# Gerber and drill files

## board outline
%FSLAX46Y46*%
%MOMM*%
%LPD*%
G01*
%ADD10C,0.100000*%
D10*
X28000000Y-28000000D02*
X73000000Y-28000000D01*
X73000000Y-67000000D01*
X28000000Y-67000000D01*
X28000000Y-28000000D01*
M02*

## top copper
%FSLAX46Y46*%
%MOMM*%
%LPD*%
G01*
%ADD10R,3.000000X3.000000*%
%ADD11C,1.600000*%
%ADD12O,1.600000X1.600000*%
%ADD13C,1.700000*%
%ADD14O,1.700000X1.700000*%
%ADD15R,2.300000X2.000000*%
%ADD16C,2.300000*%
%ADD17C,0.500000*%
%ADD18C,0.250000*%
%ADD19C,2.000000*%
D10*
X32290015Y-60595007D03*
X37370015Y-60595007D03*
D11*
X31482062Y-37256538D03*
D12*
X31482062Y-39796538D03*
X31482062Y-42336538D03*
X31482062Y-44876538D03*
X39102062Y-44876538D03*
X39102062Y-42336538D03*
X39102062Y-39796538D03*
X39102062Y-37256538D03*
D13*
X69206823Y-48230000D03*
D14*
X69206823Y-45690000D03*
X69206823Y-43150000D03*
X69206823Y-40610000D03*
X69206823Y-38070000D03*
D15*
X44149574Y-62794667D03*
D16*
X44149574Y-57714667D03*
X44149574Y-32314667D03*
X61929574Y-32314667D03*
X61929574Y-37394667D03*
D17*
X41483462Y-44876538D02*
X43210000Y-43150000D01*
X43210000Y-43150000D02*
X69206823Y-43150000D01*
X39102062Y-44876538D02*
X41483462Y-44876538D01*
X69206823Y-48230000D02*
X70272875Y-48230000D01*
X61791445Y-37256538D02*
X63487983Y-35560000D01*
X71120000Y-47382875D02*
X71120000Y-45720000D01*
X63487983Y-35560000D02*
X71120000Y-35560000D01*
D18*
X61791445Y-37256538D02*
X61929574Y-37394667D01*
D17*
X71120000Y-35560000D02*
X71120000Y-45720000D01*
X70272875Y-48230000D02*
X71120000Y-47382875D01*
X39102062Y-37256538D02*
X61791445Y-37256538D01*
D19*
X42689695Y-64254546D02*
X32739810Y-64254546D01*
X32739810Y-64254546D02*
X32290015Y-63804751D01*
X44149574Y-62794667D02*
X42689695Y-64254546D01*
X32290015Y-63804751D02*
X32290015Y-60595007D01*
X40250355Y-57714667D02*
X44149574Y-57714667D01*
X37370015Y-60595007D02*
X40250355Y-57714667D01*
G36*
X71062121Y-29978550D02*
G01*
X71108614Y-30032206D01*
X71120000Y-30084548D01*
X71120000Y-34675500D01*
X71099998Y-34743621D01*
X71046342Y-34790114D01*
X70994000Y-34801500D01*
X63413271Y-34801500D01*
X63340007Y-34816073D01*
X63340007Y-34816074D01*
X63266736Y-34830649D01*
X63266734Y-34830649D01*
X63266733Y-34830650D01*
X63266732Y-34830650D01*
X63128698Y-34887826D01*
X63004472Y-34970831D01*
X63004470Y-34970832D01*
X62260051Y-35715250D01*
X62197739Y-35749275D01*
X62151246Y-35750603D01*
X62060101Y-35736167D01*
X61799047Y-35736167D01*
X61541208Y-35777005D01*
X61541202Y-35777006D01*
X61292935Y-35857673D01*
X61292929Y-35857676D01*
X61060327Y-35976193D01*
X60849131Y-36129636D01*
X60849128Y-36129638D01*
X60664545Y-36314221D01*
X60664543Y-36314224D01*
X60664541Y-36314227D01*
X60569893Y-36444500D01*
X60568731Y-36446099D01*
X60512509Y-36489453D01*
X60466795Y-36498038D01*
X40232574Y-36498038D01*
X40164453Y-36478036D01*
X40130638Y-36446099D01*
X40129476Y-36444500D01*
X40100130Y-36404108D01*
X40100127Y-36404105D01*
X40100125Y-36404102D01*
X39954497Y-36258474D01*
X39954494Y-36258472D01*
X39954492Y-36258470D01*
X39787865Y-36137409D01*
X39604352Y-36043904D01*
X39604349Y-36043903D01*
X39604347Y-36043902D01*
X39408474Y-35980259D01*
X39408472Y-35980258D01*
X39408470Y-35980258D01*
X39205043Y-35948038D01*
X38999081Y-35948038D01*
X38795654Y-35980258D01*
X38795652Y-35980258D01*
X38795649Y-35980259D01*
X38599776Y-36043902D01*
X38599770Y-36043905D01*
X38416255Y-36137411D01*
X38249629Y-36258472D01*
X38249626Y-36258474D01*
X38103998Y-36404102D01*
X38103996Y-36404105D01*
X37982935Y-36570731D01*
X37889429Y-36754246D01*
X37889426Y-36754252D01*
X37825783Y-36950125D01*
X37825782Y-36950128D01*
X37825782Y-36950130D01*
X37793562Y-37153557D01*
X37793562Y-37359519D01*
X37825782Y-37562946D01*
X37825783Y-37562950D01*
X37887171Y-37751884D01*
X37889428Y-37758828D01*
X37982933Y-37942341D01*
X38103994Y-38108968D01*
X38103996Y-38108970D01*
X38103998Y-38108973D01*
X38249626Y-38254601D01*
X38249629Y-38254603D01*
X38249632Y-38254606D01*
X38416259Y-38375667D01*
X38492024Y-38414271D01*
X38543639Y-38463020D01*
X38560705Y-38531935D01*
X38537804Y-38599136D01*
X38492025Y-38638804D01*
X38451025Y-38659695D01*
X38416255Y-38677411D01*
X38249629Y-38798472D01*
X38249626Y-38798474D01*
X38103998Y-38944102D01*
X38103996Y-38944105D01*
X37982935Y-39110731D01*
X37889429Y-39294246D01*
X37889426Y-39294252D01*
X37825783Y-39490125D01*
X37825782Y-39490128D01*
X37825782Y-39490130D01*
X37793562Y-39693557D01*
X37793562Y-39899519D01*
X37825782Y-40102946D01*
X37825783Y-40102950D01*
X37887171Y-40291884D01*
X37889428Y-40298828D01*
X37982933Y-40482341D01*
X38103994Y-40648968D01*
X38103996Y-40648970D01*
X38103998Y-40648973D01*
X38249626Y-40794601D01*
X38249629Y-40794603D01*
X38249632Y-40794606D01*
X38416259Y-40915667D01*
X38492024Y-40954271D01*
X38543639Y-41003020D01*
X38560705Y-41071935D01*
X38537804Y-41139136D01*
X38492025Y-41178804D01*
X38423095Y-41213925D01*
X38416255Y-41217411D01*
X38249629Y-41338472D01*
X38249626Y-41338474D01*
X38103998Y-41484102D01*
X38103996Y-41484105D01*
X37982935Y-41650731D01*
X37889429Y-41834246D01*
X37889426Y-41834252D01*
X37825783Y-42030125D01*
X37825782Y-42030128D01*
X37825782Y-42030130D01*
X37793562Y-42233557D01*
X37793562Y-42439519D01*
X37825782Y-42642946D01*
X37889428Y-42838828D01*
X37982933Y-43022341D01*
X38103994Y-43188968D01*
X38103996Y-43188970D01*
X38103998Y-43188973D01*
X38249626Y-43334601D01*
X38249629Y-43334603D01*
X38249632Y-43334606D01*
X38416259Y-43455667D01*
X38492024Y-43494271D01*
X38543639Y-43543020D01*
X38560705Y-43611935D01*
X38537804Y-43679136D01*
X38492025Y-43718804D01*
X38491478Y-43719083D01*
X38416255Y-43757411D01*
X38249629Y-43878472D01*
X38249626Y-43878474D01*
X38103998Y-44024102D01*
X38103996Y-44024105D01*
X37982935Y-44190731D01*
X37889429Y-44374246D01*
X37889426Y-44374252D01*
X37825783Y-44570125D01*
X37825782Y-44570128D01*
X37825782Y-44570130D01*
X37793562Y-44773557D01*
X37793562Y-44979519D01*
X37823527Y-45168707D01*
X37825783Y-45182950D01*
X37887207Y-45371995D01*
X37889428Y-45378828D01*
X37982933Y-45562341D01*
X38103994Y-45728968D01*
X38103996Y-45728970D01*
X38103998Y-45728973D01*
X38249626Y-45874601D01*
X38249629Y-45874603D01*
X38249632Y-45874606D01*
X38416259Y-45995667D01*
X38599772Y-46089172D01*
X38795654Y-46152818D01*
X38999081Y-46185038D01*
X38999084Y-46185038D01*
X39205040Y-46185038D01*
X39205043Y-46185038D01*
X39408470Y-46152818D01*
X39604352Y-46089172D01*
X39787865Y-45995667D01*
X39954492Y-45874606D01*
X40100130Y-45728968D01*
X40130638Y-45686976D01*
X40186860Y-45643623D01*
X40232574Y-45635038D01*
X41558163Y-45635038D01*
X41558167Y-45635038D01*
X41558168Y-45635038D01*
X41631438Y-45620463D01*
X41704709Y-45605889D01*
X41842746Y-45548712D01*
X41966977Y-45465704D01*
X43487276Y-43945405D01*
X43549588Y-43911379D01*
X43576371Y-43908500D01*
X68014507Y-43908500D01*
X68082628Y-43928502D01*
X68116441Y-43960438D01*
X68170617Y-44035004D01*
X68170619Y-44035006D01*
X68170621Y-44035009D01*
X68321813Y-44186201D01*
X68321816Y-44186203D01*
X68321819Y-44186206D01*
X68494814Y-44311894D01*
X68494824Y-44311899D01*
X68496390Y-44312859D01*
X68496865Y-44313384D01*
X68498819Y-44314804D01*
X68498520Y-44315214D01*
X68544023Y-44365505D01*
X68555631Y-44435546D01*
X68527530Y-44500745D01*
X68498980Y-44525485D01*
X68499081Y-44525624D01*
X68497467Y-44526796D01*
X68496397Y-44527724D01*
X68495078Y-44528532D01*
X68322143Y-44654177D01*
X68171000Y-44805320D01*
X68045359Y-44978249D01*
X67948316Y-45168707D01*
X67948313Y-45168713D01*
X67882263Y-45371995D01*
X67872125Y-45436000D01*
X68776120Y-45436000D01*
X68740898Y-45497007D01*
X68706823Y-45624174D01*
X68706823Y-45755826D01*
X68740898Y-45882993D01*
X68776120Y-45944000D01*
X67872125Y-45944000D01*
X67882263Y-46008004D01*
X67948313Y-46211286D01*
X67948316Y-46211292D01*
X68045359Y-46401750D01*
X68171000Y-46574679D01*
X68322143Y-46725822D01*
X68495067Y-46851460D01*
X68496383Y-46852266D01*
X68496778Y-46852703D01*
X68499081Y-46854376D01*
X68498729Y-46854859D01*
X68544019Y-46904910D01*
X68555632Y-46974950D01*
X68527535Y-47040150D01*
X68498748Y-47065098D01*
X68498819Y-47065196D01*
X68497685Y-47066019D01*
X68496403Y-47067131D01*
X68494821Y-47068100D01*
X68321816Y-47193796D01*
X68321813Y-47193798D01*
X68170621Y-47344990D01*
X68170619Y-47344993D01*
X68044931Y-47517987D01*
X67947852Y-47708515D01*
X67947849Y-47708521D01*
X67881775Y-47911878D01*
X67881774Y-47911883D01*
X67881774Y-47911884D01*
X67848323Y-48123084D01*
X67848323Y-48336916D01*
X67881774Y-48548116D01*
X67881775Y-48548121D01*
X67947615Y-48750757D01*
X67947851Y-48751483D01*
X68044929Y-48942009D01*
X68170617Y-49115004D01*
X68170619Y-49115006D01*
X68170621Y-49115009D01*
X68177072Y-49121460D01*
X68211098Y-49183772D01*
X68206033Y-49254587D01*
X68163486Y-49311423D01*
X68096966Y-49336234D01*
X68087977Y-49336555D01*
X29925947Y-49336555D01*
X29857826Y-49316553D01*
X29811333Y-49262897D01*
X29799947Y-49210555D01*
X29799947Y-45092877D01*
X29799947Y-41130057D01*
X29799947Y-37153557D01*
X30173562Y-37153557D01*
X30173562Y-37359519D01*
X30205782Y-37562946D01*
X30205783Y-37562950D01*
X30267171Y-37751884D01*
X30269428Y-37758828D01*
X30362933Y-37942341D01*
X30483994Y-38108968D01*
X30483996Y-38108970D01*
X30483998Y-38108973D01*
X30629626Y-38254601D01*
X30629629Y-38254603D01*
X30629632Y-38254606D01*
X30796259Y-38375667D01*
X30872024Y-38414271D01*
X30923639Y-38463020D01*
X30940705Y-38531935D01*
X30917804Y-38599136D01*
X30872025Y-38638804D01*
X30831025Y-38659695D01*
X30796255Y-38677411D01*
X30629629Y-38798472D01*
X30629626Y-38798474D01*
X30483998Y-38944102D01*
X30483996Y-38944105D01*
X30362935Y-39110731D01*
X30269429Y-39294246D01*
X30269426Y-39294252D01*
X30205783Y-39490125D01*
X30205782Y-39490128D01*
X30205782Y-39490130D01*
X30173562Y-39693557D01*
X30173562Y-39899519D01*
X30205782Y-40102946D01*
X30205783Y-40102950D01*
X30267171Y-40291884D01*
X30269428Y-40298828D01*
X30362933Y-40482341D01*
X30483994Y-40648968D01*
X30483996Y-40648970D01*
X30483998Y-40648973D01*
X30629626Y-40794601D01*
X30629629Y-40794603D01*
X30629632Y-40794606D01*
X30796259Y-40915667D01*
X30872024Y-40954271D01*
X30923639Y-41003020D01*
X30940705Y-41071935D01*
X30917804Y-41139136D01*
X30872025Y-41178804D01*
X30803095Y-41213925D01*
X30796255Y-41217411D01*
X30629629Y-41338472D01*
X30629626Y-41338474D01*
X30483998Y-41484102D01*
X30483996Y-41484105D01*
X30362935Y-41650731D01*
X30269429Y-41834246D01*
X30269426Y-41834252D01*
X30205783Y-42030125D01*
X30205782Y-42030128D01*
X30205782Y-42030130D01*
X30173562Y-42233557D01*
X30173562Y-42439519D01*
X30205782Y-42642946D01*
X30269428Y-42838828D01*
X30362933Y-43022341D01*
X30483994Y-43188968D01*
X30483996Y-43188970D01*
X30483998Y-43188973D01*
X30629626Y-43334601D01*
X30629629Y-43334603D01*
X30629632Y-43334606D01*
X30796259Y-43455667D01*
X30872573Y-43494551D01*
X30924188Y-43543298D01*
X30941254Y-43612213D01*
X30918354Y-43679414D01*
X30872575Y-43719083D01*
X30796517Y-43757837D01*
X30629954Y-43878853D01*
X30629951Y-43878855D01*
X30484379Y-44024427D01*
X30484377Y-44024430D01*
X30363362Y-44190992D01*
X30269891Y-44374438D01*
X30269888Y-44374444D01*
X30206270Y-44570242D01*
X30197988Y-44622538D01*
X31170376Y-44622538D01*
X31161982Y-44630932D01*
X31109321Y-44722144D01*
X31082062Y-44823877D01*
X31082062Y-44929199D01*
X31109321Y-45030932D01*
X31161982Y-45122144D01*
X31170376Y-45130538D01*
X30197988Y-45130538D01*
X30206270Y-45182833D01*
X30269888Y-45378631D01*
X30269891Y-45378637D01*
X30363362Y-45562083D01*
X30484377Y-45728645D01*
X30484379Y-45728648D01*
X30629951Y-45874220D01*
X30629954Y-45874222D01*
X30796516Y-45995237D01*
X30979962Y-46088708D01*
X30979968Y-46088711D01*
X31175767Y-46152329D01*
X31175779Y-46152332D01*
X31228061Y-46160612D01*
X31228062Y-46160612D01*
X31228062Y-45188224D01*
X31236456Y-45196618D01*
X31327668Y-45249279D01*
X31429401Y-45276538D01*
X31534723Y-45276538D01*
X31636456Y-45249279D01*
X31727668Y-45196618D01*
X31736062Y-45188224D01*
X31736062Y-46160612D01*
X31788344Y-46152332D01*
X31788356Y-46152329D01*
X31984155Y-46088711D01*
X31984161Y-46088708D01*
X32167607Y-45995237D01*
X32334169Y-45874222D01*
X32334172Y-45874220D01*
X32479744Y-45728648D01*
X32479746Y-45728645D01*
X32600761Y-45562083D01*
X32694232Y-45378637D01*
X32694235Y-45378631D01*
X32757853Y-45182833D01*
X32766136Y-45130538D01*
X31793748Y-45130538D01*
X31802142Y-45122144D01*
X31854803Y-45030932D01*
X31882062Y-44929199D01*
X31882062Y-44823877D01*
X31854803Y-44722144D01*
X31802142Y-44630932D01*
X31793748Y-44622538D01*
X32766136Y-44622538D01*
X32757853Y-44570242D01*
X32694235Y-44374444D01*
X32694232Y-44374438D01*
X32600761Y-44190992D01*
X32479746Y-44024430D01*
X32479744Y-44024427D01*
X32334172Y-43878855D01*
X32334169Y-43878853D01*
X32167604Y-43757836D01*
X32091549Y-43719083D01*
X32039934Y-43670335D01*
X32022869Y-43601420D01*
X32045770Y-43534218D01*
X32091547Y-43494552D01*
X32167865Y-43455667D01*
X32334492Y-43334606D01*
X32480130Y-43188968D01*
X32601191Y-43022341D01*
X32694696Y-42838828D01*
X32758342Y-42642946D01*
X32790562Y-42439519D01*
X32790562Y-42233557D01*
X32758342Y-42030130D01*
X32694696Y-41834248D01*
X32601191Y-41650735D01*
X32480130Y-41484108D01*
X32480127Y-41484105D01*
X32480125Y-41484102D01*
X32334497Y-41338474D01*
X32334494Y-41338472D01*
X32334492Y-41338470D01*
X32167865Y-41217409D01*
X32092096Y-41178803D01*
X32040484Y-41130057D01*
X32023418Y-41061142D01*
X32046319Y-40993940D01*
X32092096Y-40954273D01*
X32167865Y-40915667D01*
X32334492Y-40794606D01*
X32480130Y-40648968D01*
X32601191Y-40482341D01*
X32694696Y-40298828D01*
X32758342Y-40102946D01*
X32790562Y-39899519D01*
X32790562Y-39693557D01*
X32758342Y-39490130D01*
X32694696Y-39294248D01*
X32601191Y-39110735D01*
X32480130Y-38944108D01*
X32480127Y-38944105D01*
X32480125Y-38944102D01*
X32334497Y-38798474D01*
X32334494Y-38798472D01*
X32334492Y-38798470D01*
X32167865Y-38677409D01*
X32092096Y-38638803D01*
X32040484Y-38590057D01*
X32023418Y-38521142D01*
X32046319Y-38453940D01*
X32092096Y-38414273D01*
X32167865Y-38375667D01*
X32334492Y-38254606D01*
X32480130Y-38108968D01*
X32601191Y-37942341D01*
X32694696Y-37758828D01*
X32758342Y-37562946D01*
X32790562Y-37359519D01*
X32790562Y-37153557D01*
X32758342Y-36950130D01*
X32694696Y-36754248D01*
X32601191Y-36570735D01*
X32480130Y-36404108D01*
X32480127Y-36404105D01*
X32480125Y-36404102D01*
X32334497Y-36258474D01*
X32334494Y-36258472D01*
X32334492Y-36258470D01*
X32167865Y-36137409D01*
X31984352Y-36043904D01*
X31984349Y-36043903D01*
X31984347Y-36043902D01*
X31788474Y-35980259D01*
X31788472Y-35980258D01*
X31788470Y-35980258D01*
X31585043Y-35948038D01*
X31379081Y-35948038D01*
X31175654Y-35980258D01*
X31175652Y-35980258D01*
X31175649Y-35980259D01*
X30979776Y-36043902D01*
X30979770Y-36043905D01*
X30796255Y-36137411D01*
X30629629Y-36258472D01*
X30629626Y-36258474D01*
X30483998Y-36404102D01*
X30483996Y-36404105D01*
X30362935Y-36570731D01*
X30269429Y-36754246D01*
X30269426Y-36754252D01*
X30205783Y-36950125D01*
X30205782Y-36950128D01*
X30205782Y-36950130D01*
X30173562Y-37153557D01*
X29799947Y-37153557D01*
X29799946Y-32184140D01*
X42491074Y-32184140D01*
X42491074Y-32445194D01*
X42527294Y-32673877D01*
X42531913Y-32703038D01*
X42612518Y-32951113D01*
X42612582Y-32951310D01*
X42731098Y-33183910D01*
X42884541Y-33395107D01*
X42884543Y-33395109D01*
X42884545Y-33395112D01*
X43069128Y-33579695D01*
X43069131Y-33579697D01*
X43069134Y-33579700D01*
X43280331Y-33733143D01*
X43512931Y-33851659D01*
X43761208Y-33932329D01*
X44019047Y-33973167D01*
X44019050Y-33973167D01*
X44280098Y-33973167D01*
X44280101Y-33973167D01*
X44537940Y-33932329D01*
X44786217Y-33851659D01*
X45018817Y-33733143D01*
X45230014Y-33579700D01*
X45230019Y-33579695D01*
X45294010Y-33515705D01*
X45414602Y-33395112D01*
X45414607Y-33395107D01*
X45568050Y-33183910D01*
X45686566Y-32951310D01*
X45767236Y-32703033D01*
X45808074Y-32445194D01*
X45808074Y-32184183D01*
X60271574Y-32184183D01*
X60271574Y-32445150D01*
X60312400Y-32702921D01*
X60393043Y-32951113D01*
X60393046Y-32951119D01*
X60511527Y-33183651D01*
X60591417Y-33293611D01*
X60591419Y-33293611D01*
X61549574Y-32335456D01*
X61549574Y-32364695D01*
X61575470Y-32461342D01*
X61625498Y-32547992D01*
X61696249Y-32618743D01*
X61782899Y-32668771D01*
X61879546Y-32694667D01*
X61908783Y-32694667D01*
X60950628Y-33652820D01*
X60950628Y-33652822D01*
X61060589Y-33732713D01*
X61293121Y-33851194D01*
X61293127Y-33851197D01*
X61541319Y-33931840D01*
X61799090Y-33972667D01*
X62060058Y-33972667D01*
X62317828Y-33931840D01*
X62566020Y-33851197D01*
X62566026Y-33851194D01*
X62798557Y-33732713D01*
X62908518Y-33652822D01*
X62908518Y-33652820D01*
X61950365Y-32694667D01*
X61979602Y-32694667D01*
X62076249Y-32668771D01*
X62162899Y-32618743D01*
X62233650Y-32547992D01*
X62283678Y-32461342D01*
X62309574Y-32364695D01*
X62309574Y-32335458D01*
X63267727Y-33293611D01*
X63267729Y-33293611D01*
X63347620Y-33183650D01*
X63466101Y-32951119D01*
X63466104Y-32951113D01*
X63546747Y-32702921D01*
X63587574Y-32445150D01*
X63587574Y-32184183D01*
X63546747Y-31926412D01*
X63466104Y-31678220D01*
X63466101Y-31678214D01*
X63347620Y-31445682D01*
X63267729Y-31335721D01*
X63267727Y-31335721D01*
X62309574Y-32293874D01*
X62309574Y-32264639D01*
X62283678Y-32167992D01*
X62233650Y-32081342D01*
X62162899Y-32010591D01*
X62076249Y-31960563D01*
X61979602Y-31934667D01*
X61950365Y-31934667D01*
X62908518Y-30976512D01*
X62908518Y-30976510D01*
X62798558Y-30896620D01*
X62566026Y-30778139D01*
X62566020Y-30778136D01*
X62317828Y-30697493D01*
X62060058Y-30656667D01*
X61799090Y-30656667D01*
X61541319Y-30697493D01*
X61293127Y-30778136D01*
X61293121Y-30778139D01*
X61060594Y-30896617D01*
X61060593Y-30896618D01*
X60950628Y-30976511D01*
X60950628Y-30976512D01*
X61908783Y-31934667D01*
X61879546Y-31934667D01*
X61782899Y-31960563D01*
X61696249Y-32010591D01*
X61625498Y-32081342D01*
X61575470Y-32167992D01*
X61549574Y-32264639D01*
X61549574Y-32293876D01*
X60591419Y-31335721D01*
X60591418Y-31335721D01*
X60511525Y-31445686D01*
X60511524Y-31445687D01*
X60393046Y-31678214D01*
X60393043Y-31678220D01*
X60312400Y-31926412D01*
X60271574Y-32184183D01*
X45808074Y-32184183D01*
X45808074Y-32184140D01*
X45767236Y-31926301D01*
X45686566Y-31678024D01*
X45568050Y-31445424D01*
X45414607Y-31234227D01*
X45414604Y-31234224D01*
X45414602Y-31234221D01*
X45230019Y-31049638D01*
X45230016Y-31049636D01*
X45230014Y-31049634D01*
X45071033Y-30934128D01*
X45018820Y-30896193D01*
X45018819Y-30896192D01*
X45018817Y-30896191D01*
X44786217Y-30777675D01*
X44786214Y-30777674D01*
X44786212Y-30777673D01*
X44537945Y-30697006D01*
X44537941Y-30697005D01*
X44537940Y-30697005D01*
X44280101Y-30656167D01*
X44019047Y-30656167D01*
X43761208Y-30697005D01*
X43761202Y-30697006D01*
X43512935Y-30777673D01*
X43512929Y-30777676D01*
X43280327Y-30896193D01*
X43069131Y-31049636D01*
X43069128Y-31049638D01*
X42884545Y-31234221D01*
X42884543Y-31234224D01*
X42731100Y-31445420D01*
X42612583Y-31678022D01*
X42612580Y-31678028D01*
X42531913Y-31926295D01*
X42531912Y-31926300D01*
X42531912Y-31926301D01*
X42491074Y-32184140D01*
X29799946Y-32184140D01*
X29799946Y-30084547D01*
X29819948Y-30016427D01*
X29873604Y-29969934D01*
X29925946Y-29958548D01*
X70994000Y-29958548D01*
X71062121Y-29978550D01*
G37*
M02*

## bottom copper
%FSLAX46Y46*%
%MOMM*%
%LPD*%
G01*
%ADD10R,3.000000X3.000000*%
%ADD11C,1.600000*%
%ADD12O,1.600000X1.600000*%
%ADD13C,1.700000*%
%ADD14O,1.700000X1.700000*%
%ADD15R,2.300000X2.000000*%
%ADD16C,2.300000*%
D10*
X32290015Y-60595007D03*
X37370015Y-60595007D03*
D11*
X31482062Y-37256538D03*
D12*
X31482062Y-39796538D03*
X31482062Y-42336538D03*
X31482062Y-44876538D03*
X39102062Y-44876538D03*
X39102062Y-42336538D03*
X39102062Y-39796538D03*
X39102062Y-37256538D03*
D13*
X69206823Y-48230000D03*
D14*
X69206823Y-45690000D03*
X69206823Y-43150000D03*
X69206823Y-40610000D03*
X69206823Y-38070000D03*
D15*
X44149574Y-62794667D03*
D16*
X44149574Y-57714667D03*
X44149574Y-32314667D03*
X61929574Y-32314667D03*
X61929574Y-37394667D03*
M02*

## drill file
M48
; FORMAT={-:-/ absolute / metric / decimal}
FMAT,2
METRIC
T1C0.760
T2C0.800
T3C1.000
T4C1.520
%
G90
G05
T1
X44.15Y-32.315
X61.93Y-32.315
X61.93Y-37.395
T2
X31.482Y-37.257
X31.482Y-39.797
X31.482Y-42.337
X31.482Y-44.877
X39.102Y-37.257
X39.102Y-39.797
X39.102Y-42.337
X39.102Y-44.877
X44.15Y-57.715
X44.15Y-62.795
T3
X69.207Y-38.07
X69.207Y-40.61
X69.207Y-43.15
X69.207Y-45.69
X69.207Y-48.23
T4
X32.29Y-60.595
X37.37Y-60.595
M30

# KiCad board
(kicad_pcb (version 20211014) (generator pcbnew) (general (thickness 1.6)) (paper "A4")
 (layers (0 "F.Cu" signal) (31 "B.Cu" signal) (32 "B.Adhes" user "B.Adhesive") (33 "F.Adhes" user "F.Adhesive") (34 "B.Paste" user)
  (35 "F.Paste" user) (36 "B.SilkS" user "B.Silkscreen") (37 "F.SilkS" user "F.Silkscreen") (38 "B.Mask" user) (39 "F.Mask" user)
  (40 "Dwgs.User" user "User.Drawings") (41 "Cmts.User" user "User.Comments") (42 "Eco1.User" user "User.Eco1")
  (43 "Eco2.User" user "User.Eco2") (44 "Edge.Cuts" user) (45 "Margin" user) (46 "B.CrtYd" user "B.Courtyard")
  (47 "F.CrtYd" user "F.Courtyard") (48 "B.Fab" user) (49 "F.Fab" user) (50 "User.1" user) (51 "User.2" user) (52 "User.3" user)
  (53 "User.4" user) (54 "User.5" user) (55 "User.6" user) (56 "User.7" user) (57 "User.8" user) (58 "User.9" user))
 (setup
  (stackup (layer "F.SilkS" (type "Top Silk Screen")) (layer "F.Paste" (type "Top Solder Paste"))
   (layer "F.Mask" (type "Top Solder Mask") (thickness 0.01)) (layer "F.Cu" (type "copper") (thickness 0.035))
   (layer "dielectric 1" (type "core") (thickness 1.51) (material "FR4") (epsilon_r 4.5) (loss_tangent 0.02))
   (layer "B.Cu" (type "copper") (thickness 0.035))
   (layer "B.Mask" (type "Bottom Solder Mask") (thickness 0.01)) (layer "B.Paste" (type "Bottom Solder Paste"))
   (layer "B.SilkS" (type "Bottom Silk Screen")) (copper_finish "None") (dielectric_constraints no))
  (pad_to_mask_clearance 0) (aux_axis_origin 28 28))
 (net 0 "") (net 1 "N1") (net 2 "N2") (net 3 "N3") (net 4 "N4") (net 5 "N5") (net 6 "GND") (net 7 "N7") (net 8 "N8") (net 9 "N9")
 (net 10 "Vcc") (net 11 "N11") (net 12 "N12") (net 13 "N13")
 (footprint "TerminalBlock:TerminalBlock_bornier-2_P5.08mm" (layer "F.Cu") (at 32.290015 60.595007)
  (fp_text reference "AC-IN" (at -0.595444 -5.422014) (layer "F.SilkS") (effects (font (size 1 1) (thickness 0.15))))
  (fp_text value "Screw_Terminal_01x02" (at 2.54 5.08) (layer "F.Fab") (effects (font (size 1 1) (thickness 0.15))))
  (pad "1" thru_hole rect (at 0 0) (size 3 3) (drill 1.52) (layers *.Cu *.Mask) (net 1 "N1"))
  (pad "2" thru_hole rect (at 5.08 0) (size 3 3) (drill 1.52) (layers *.Cu *.Mask) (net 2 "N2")))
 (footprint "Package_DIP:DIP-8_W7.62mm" (layer "F.Cu") (at 31.482062 37.256538)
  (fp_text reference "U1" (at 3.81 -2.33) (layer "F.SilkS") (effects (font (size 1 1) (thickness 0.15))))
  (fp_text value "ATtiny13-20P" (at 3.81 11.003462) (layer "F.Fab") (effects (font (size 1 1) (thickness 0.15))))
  (pad "1" thru_hole circle (at 0 0) (size 1.6 1.6) (drill 0.8) (layers *.Cu *.Mask) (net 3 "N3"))
  (pad "2" thru_hole oval (at 0 2.54) (size 1.6 1.6) (drill 0.8) (layers *.Cu *.Mask) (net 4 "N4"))
  (pad "3" thru_hole oval (at 0 5.08) (size 1.6 1.6) (drill 0.8) (layers *.Cu *.Mask) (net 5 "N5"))
  (pad "4" thru_hole oval (at 0 7.62) (size 1.6 1.6) (drill 0.8) (layers *.Cu *.Mask) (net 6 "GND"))
  (pad "5" thru_hole oval (at 7.62 7.62) (size 1.6 1.6) (drill 0.8) (layers *.Cu *.Mask) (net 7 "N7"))
  (pad "6" thru_hole oval (at 7.62 5.08) (size 1.6 1.6) (drill 0.8) (layers *.Cu *.Mask) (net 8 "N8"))
  (pad "7" thru_hole oval (at 7.62 2.54) (size 1.6 1.6) (drill 0.8) (layers *.Cu *.Mask) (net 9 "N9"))
  (pad "8" thru_hole oval (at 7.62 0) (size 1.6 1.6) (drill 0.8) (layers *.Cu *.Mask) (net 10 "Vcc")))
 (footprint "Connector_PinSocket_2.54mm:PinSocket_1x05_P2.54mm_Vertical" (layer "F.Cu") (at 69.206823 48.23 180)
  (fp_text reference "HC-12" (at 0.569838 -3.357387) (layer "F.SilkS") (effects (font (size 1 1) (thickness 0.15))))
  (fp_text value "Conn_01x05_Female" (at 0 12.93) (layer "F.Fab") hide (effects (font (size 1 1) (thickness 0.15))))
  (pad "1" thru_hole circle (at 0 0 180) (size 1.7 1.7) (drill 1) (layers *.Cu *.Mask) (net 10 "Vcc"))
  (pad "2" thru_hole oval (at 0 2.54 180) (size 1.7 1.7) (drill 1) (layers *.Cu *.Mask) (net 6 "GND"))
  (pad "3" thru_hole oval (at 0 5.08 180) (size 1.7 1.7) (drill 1) (layers *.Cu *.Mask) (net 7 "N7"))
  (pad "4" thru_hole oval (at 0 7.62 180) (size 1.7 1.7) (drill 1) (layers *.Cu *.Mask) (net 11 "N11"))
  (pad "5" thru_hole oval (at 0 10.16 180) (size 1.7 1.7) (drill 1) (layers *.Cu *.Mask) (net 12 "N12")))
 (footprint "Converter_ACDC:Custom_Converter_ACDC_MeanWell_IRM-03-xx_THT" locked (layer "B.Cu") (at 44.149574 62.794667)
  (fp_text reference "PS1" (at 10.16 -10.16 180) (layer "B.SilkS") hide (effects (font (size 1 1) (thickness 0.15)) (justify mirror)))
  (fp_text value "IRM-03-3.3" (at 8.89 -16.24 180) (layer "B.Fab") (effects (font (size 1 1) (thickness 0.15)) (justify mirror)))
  (pad "1" thru_hole rect locked (at 0 0) (size 2.3 2) (drill 0.8) (layers *.Cu *.Mask) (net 1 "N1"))
  (pad "3" thru_hole circle locked (at 0 -5.08) (size 2.3 2.3) (drill 0.8) (layers *.Cu *.Mask) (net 2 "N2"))
  (pad "5" thru_hole circle locked (at 0 -30.48) (size 2.3 2.3) (drill 0.76) (layers *.Cu *.Mask) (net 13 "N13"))
  (pad "14" thru_hole circle locked (at 17.78 -30.48) (size 2.3 2.3) (drill 0.76) (layers *.Cu *.Mask) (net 6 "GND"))
  (pad "16" thru_hole circle locked (at 17.78 -25.4) (size 2.3 2.3) (drill 0.76) (layers *.Cu *.Mask) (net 10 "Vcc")))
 (gr_rect (start 28 28) (end 73 67) (layer "Edge.Cuts") (width 0.1) (fill none))
 (segment (start 41.483462 44.876538) (end 43.21 43.15) (width 0.5) (layer "F.Cu") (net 7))
 (segment (start 43.21 43.15) (end 69.206823 43.15) (width 0.5) (layer "F.Cu") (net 7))
 (segment (start 39.102062 44.876538) (end 41.483462 44.876538) (width 0.5) (layer "F.Cu") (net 7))
 (segment (start 69.206823 48.23) (end 70.272875 48.23) (width 0.5) (layer "F.Cu") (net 10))
 (segment (start 61.791445 37.256538) (end 63.487983 35.56) (width 0.5) (layer "F.Cu") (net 10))
 (segment (start 71.12 47.382875) (end 71.12 45.72) (width 0.5) (layer "F.Cu") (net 10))
 (segment (start 63.487983 35.56) (end 71.12 35.56) (width 0.5) (layer "F.Cu") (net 10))
 (segment (start 61.791445 37.256538) (end 61.929574 37.394667) (width 0.25) (layer "F.Cu") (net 10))
 (segment (start 71.12 35.56) (end 71.12 45.72) (width 0.5) (layer "F.Cu") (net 10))
 (segment (start 70.272875 48.23) (end 71.12 47.382875) (width 0.5) (layer "F.Cu") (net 10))
 (segment (start 39.102062 37.256538) (end 61.791445 37.256538) (width 0.5) (layer "F.Cu") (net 10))
 (segment (start 42.689695 64.254546) (end 32.73981 64.254546) (width 2) (layer "F.Cu") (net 1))
 (segment (start 32.73981 64.254546) (end 32.290015 63.804751) (width 2) (layer "F.Cu") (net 1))
 (segment (start 44.149574 62.794667) (end 42.689695 64.254546) (width 2) (layer "F.Cu") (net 1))
 (segment (start 32.290015 63.804751) (end 32.290015 60.595007) (width 2) (layer "F.Cu") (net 1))
 (segment (start 40.250355 57.714667) (end 44.149574 57.714667) (width 2) (layer "F.Cu") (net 2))
 (segment (start 37.370015 60.595007) (end 40.250355 57.714667) (width 2) (layer "F.Cu") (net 2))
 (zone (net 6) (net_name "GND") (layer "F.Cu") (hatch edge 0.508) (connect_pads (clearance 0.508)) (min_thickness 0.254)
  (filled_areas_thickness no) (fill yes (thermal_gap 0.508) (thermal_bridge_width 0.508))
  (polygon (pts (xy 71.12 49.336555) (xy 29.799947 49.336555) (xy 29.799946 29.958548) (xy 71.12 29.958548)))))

